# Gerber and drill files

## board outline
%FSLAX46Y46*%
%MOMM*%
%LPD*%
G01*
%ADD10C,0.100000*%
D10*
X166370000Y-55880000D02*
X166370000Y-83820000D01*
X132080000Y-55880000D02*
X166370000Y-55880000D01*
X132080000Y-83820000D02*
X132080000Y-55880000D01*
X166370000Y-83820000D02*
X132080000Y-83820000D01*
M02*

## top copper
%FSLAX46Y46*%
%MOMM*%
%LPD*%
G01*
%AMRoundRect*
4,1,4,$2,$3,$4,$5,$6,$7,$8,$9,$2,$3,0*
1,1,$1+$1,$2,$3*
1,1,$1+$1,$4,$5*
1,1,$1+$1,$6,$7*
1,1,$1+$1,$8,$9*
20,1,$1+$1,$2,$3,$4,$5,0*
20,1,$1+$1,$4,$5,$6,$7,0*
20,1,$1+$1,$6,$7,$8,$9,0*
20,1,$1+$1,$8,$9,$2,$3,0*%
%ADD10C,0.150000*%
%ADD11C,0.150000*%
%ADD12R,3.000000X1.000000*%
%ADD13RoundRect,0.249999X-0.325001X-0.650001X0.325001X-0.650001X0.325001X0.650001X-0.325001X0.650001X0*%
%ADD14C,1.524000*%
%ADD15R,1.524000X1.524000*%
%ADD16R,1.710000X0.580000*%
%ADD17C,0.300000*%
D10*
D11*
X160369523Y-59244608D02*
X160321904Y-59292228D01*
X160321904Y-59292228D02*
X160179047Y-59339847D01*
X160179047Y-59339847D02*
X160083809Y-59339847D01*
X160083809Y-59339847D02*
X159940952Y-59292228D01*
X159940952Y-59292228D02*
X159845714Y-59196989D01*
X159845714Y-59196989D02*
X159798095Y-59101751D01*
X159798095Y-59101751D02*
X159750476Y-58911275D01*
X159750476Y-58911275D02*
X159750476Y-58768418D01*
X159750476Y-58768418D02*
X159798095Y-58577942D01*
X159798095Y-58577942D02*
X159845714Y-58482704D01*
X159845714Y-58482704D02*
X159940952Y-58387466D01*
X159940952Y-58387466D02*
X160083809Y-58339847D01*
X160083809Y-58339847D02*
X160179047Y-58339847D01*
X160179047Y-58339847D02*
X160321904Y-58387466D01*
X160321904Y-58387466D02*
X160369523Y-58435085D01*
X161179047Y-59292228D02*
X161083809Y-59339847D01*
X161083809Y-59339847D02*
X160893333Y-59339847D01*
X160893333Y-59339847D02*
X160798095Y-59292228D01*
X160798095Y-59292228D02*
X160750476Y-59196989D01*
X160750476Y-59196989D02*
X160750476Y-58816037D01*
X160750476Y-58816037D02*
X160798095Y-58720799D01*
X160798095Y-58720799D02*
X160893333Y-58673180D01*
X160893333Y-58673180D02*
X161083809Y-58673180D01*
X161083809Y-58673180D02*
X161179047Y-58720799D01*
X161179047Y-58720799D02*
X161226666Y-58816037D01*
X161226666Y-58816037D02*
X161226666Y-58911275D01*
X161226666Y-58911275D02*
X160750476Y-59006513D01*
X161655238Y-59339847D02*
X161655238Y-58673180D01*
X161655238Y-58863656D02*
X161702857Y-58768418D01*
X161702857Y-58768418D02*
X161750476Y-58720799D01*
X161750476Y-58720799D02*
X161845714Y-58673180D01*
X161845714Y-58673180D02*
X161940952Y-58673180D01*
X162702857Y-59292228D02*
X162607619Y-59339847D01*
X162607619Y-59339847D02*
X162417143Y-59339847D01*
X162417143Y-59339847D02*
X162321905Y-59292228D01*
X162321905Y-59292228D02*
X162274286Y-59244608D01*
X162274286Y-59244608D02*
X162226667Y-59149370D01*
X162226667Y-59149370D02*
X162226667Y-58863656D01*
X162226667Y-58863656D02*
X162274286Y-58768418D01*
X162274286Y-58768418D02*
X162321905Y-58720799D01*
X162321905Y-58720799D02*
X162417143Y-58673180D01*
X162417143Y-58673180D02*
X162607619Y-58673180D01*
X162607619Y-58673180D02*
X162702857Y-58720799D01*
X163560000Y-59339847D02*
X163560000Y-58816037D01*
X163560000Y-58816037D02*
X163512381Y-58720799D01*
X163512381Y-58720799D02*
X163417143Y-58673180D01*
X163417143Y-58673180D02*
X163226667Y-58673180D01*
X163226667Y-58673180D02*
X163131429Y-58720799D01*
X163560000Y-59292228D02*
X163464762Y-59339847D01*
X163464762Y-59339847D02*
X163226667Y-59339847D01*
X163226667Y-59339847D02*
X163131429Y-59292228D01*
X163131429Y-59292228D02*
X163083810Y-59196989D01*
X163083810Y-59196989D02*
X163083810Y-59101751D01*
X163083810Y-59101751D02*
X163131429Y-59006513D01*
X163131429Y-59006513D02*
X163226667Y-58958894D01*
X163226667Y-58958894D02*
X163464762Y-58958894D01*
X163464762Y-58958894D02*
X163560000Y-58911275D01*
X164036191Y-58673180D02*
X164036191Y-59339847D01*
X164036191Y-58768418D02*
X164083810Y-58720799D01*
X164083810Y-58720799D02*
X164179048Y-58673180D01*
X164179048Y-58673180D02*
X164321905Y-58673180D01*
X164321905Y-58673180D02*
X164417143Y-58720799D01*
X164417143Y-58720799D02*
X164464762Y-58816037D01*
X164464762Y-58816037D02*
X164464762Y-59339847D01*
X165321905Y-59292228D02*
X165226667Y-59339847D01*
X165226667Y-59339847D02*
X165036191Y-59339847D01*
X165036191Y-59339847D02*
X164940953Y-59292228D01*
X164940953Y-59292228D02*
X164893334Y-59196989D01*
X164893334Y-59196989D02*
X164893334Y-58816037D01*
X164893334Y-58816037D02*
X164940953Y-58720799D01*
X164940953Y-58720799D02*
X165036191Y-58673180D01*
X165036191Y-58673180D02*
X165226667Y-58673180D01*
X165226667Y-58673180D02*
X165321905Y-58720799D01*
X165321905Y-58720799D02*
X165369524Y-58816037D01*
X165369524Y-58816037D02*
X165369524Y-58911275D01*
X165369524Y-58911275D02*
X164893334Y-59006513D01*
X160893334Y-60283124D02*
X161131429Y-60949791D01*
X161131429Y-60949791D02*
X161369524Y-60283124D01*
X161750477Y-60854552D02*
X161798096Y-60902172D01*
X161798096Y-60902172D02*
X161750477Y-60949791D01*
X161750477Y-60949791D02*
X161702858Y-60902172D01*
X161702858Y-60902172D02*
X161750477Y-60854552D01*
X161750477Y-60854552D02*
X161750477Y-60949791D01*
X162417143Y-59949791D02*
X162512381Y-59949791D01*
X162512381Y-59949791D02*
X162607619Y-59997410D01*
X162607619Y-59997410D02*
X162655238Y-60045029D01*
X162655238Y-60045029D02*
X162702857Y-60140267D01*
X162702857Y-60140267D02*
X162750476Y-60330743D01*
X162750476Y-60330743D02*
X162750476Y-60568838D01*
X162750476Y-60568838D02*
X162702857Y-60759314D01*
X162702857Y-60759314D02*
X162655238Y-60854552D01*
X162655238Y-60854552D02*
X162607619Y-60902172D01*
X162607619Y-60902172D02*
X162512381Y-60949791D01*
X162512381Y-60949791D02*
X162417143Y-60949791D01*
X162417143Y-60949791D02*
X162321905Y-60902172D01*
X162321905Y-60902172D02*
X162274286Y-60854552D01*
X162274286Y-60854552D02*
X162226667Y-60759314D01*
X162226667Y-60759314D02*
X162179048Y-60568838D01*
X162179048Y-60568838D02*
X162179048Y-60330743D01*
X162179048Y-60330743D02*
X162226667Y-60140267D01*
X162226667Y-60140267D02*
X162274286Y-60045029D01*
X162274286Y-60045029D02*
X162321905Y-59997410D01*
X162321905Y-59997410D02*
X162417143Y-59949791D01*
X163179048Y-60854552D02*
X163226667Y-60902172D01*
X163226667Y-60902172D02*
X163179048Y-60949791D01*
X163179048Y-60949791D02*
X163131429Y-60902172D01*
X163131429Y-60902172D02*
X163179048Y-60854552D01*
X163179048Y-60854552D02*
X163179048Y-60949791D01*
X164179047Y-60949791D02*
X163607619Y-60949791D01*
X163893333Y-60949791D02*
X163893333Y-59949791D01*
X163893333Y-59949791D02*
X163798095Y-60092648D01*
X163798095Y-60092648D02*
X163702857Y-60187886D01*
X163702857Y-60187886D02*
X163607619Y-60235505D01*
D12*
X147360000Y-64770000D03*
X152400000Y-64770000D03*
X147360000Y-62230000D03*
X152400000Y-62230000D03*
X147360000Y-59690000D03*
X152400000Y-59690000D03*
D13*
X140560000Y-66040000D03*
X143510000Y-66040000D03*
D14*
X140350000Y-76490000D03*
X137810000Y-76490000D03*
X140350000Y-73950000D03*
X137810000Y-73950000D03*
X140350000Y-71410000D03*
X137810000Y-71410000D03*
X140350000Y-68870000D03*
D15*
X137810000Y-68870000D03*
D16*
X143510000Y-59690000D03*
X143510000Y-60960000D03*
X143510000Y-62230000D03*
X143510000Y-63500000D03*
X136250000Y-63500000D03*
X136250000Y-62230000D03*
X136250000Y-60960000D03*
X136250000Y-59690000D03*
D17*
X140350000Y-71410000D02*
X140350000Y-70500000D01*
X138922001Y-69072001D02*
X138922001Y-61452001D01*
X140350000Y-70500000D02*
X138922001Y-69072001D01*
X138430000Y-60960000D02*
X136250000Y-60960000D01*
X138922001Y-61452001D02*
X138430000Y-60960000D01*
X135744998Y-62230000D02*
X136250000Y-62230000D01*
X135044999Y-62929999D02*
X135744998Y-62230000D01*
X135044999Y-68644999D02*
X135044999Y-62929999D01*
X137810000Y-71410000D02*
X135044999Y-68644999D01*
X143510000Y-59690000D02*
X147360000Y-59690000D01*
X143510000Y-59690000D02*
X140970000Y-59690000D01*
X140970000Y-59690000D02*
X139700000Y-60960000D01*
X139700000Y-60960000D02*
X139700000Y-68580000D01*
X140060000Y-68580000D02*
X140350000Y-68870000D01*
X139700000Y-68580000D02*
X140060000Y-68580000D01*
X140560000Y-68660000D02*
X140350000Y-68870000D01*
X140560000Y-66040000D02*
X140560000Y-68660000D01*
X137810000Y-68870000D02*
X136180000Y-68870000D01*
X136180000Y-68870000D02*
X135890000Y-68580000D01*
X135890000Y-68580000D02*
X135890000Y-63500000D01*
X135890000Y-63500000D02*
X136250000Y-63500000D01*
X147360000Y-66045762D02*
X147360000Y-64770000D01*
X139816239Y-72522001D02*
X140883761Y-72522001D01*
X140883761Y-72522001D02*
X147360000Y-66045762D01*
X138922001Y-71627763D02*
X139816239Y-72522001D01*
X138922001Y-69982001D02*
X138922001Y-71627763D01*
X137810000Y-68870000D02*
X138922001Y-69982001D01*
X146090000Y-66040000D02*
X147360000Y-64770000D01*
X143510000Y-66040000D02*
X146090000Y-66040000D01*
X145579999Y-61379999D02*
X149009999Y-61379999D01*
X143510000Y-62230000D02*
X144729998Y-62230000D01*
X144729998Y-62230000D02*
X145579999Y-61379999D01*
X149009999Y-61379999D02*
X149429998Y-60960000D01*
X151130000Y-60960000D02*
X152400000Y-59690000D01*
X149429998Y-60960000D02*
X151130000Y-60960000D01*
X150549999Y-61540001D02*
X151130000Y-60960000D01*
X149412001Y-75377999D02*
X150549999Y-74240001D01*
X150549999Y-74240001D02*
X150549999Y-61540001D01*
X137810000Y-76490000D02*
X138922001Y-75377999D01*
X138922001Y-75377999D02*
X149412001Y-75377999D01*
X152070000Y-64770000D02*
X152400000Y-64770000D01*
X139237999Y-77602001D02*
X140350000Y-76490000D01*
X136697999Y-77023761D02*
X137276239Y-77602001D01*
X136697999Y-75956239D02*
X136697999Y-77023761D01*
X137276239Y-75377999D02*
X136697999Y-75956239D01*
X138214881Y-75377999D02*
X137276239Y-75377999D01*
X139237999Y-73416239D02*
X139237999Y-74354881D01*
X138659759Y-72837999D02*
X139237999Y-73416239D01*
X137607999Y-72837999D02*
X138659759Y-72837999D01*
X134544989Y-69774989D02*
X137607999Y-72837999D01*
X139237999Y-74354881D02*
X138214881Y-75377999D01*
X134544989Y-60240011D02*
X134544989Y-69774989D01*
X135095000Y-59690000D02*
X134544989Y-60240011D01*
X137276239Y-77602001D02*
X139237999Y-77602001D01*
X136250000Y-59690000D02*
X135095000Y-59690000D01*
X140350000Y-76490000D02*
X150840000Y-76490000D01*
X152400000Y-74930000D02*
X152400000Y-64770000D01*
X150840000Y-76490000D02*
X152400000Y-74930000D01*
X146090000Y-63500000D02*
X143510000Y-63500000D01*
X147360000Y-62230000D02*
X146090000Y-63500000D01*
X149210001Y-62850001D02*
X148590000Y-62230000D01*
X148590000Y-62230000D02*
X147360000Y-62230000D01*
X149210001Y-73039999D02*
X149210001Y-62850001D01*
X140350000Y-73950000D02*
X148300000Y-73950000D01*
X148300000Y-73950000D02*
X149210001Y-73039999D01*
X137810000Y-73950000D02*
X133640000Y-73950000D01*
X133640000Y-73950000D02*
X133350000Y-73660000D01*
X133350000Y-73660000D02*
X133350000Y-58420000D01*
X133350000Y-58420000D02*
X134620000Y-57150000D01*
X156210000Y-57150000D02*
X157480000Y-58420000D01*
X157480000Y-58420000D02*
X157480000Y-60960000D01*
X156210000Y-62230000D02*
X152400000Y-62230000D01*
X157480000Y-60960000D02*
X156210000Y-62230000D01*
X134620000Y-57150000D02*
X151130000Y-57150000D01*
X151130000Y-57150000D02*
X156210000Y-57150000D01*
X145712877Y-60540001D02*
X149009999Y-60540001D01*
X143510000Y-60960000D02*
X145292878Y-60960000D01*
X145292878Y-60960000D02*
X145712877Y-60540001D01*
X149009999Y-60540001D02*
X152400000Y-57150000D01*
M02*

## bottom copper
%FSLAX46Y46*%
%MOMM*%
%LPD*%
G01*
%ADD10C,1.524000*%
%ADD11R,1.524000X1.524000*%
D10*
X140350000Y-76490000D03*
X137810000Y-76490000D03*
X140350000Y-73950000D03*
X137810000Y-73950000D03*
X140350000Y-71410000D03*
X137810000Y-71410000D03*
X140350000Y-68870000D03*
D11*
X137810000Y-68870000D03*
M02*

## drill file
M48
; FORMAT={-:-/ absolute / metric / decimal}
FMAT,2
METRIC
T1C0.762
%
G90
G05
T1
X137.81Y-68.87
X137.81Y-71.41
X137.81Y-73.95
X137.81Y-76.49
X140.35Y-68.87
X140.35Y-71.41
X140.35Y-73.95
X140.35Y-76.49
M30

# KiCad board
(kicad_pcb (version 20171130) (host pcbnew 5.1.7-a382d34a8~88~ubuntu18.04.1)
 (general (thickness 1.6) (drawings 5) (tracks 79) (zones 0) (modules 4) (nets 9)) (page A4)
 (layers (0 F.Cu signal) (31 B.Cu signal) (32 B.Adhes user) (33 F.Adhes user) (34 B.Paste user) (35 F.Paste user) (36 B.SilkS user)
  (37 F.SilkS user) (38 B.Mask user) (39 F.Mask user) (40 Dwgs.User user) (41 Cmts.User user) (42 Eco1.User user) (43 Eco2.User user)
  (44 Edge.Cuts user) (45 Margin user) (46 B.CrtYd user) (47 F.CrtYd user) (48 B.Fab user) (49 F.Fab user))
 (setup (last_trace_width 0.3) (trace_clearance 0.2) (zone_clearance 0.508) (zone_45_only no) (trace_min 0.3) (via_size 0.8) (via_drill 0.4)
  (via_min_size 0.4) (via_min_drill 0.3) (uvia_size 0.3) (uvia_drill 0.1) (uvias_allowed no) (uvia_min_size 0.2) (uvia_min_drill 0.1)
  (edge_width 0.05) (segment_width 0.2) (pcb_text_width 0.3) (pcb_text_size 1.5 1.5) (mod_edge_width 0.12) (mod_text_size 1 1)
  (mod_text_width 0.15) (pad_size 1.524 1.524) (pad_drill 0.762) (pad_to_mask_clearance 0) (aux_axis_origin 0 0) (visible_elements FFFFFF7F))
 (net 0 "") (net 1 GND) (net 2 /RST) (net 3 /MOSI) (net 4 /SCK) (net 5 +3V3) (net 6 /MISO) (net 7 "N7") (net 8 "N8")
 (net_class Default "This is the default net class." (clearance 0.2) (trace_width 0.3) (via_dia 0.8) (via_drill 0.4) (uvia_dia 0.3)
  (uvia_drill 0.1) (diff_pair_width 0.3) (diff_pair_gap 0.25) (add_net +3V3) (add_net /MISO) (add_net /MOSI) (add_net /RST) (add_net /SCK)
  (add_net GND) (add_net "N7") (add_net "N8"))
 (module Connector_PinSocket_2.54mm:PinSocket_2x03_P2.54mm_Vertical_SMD (layer F.Cu) (at 149.88 62.23)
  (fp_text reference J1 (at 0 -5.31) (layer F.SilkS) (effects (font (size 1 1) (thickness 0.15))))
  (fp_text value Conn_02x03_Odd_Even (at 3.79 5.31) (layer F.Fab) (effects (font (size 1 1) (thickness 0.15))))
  (pad 6 smd rect (at -2.52 2.54) (size 3 1) (layers F.Cu F.Paste F.Mask) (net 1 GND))
  (pad 5 smd rect (at 2.52 2.54) (size 3 1) (layers F.Cu F.Paste F.Mask) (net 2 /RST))
  (pad 4 smd rect (at -2.52 0) (size 3 1) (layers F.Cu F.Paste F.Mask) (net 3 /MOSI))
  (pad 3 smd rect (at 2.52 0) (size 3 1) (layers F.Cu F.Paste F.Mask) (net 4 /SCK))
  (pad 2 smd rect (at -2.52 -2.54) (size 3 1) (layers F.Cu F.Paste F.Mask) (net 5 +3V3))
  (pad 1 smd rect (at 2.52 -2.54) (size 3 1) (layers F.Cu F.Paste F.Mask) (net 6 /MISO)))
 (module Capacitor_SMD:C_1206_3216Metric (layer F.Cu) (at 142.035 66.04)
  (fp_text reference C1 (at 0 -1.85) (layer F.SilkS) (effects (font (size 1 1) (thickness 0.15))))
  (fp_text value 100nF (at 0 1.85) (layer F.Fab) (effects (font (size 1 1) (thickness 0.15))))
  (pad 1 smd roundrect (at -1.475 0) (size 1.15 1.8) (layers F.Cu F.Paste F.Mask) (roundrect_rratio 0.2173904347826087) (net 5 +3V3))
  (pad 2 smd roundrect (at 1.475 0) (size 1.15 1.8) (layers F.Cu F.Paste F.Mask) (roundrect_rratio 0.2173904347826087) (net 1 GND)))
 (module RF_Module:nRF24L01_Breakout (layer F.Cu) (at 137.81 68.87)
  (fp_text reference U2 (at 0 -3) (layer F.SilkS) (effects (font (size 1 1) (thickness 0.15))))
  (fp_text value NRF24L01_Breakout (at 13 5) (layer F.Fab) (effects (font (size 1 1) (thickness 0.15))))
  (pad 8 thru_hole circle (at 2.54 7.62) (size 1.524 1.524) (drill 0.762) (layers *.Cu *.Mask) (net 2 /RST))
  (pad 7 thru_hole circle (at 0 7.62) (size 1.524 1.524) (drill 0.762) (layers *.Cu *.Mask) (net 6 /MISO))
  (pad 6 thru_hole circle (at 2.54 5.08) (size 1.524 1.524) (drill 0.762) (layers *.Cu *.Mask) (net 3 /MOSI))
  (pad 5 thru_hole circle (at 0 5.08) (size 1.524 1.524) (drill 0.762) (layers *.Cu *.Mask) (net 4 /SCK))
  (pad 4 thru_hole circle (at 2.54 2.54) (size 1.524 1.524) (drill 0.762) (layers *.Cu *.Mask) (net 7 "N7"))
  (pad 3 thru_hole circle (at 0 2.54) (size 1.524 1.524) (drill 0.762) (layers *.Cu *.Mask) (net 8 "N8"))
  (pad 2 thru_hole circle (at 2.54 0) (size 1.524 1.524) (drill 0.762) (layers *.Cu *.Mask) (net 5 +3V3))
  (pad 1 thru_hole rect (at 0 0) (size 1.524 1.524) (drill 0.762) (layers *.Cu *.Mask) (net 1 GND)))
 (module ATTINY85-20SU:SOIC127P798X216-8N (layer F.Cu) (at 139.88 61.595)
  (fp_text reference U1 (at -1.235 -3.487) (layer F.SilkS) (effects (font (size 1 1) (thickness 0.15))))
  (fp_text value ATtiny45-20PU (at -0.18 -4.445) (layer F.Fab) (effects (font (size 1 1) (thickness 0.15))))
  (pad 8 smd rect (at 3.63 -1.905) (size 1.71 0.58) (layers F.Cu F.Paste F.Mask) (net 5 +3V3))
  (pad 7 smd rect (at 3.63 -0.635) (size 1.71 0.58) (layers F.Cu F.Paste F.Mask) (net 4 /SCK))
  (pad 6 smd rect (at 3.63 0.635) (size 1.71 0.58) (layers F.Cu F.Paste F.Mask) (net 6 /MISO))
  (pad 5 smd rect (at 3.63 1.905) (size 1.71 0.58) (layers F.Cu F.Paste F.Mask) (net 3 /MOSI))
  (pad 4 smd rect (at -3.63 1.905) (size 1.71 0.58) (layers F.Cu F.Paste F.Mask) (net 1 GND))
  (pad 3 smd rect (at -3.63 0.635) (size 1.71 0.58) (layers F.Cu F.Paste F.Mask) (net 8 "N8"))
  (pad 2 smd rect (at -3.63 -0.635) (size 1.71 0.58) (layers F.Cu F.Paste F.Mask) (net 7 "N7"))
  (pad 1 smd rect (at -3.63 -1.905) (size 1.71 0.58) (layers F.Cu F.Paste F.Mask) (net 2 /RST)))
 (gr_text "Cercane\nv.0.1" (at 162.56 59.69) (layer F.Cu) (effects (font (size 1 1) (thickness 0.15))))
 (gr_line (start 166.37 55.88) (end 166.37 83.82) (layer Edge.Cuts) (width 0.1))
 (gr_line (start 132.08 55.88) (end 166.37 55.88) (layer Edge.Cuts) (width 0.1))
 (gr_line (start 132.08 83.82) (end 132.08 55.88) (layer Edge.Cuts) (width 0.1))
 (gr_line (start 166.37 83.82) (end 132.08 83.82) (layer Edge.Cuts) (width 0.1))
 (segment (start 140.35 71.41) (end 140.35 70.5) (width 0.3) (layer F.Cu) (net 7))
 (segment (start 138.922001 69.072001) (end 138.922001 61.452001) (width 0.3) (layer F.Cu) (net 7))
 (segment (start 140.35 70.5) (end 138.922001 69.072001) (width 0.3) (layer F.Cu) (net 7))
 (segment (start 138.43 60.96) (end 136.25 60.96) (width 0.3) (layer F.Cu) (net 7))
 (segment (start 138.922001 61.452001) (end 138.43 60.96) (width 0.3) (layer F.Cu) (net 7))
 (segment (start 135.744998 62.23) (end 136.25 62.23) (width 0.3) (layer F.Cu) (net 8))
 (segment (start 135.044999 62.929999) (end 135.744998 62.23) (width 0.3) (layer F.Cu) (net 8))
 (segment (start 135.044999 68.644999) (end 135.044999 62.929999) (width 0.3) (layer F.Cu) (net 8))
 (segment (start 137.81 71.41) (end 135.044999 68.644999) (width 0.3) (layer F.Cu) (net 8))
 (segment (start 143.51 59.69) (end 147.36 59.69) (width 0.3) (layer F.Cu) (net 5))
 (segment (start 143.51 59.69) (end 140.97 59.69) (width 0.3) (layer F.Cu) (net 5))
 (segment (start 140.97 59.69) (end 139.7 60.96) (width 0.3) (layer F.Cu) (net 5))
 (segment (start 139.7 60.96) (end 139.7 68.58) (width 0.3) (layer F.Cu) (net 5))
 (segment (start 140.06 68.58) (end 140.35 68.87) (width 0.3) (layer F.Cu) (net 5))
 (segment (start 139.7 68.58) (end 140.06 68.58) (width 0.3) (layer F.Cu) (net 5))
 (segment (start 140.56 68.66) (end 140.35 68.87) (width 0.3) (layer F.Cu) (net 5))
 (segment (start 140.56 66.04) (end 140.56 68.66) (width 0.3) (layer F.Cu) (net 5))
 (segment (start 137.81 68.87) (end 136.18 68.87) (width 0.3) (layer F.Cu) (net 1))
 (segment (start 136.18 68.87) (end 135.89 68.58) (width 0.3) (layer F.Cu) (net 1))
 (segment (start 135.89 68.58) (end 135.89 63.5) (width 0.3) (layer F.Cu) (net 1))
 (segment (start 135.89 63.5) (end 136.25 63.5) (width 0.3) (layer F.Cu) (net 1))
 (segment (start 147.36 66.045762) (end 147.36 64.77) (width 0.3) (layer F.Cu) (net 1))
 (segment (start 139.816239 72.522001) (end 140.883761 72.522001) (width 0.3) (layer F.Cu) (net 1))
 (segment (start 140.883761 72.522001) (end 147.36 66.045762) (width 0.3) (layer F.Cu) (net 1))
 (segment (start 138.922001 71.627763) (end 139.816239 72.522001) (width 0.3) (layer F.Cu) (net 1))
 (segment (start 138.922001 69.982001) (end 138.922001 71.627763) (width 0.3) (layer F.Cu) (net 1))
 (segment (start 137.81 68.87) (end 138.922001 69.982001) (width 0.3) (layer F.Cu) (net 1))
 (segment (start 146.09 66.04) (end 147.36 64.77) (width 0.3) (layer F.Cu) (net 1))
 (segment (start 143.51 66.04) (end 146.09 66.04) (width 0.3) (layer F.Cu) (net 1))
 (segment (start 145.579999 61.379999) (end 149.009999 61.379999) (width 0.3) (layer F.Cu) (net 6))
 (segment (start 143.51 62.23) (end 144.729998 62.23) (width 0.3) (layer F.Cu) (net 6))
 (segment (start 144.729998 62.23) (end 145.579999 61.379999) (width 0.3) (layer F.Cu) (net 6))
 (segment (start 149.009999 61.379999) (end 149.429998 60.96) (width 0.3) (layer F.Cu) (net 6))
 (segment (start 151.13 60.96) (end 152.4 59.69) (width 0.3) (layer F.Cu) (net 6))
 (segment (start 149.429998 60.96) (end 151.13 60.96) (width 0.3) (layer F.Cu) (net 6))
 (segment (start 150.549999 61.540001) (end 151.13 60.96) (width 0.3) (layer F.Cu) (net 6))
 (segment (start 149.412001 75.377999) (end 150.549999 74.240001) (width 0.3) (layer F.Cu) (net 6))
 (segment (start 150.549999 74.240001) (end 150.549999 61.540001) (width 0.3) (layer F.Cu) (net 6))
 (segment (start 137.81 76.49) (end 138.922001 75.377999) (width 0.3) (layer F.Cu) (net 6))
 (segment (start 138.922001 75.377999) (end 149.412001 75.377999) (width 0.3) (layer F.Cu) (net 6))
 (segment (start 152.07 64.77) (end 152.4 64.77) (width 0.3) (layer F.Cu) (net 2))
 (segment (start 139.237999 77.602001) (end 140.35 76.49) (width 0.3) (layer F.Cu) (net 2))
 (segment (start 136.697999 77.023761) (end 137.276239 77.602001) (width 0.3) (layer F.Cu) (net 2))
 (segment (start 136.697999 75.956239) (end 136.697999 77.023761) (width 0.3) (layer F.Cu) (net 2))
 (segment (start 137.276239 75.377999) (end 136.697999 75.956239) (width 0.3) (layer F.Cu) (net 2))
 (segment (start 138.214881 75.377999) (end 137.276239 75.377999) (width 0.3) (layer F.Cu) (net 2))
 (segment (start 139.237999 73.416239) (end 139.237999 74.354881) (width 0.3) (layer F.Cu) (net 2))
 (segment (start 138.659759 72.837999) (end 139.237999 73.416239) (width 0.3) (layer F.Cu) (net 2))
 (segment (start 137.607999 72.837999) (end 138.659759 72.837999) (width 0.3) (layer F.Cu) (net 2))
 (segment (start 134.544989 69.774989) (end 137.607999 72.837999) (width 0.3) (layer F.Cu) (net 2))
 (segment (start 139.237999 74.354881) (end 138.214881 75.377999) (width 0.3) (layer F.Cu) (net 2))
 (segment (start 134.544989 60.240011) (end 134.544989 69.774989) (width 0.3) (layer F.Cu) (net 2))
 (segment (start 135.095 59.69) (end 134.544989 60.240011) (width 0.3) (layer F.Cu) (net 2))
 (segment (start 137.276239 77.602001) (end 139.237999 77.602001) (width 0.3) (layer F.Cu) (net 2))
 (segment (start 136.25 59.69) (end 135.095 59.69) (width 0.3) (layer F.Cu) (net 2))
 (segment (start 140.35 76.49) (end 150.84 76.49) (width 0.3) (layer F.Cu) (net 2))
 (segment (start 152.4 74.93) (end 152.4 64.77) (width 0.3) (layer F.Cu) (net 2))
 (segment (start 150.84 76.49) (end 152.4 74.93) (width 0.3) (layer F.Cu) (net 2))
 (segment (start 146.09 63.5) (end 143.51 63.5) (width 0.3) (layer F.Cu) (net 3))
 (segment (start 147.36 62.23) (end 146.09 63.5) (width 0.3) (layer F.Cu) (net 3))
 (segment (start 149.210001 62.850001) (end 148.59 62.23) (width 0.3) (layer F.Cu) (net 3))
 (segment (start 148.59 62.23) (end 147.36 62.23) (width 0.3) (layer F.Cu) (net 3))
 (segment (start 149.210001 73.039999) (end 149.210001 62.850001) (width 0.3) (layer F.Cu) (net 3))
 (segment (start 140.35 73.95) (end 148.3 73.95) (width 0.3) (layer F.Cu) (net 3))
 (segment (start 148.3 73.95) (end 149.210001 73.039999) (width 0.3) (layer F.Cu) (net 3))
 (segment (start 137.81 73.95) (end 133.64 73.95) (width 0.3) (layer F.Cu) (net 4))
 (segment (start 133.64 73.95) (end 133.35 73.66) (width 0.3) (layer F.Cu) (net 4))
 (segment (start 133.35 73.66) (end 133.35 58.42) (width 0.3) (layer F.Cu) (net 4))
 (segment (start 133.35 58.42) (end 134.62 57.15) (width 0.3) (layer F.Cu) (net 4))
 (segment (start 156.21 57.15) (end 157.48 58.42) (width 0.3) (layer F.Cu) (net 4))
 (segment (start 157.48 58.42) (end 157.48 60.96) (width 0.3) (layer F.Cu) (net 4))
 (segment (start 156.21 62.23) (end 152.4 62.23) (width 0.3) (layer F.Cu) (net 4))
 (segment (start 157.48 60.96) (end 156.21 62.23) (width 0.3) (layer F.Cu) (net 4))
 (segment (start 134.62 57.15) (end 151.13 57.15) (width 0.3) (layer F.Cu) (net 4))
 (segment (start 151.13 57.15) (end 156.21 57.15) (width 0.3) (layer F.Cu) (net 4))
 (segment (start 145.712877 60.540001) (end 149.009999 60.540001) (width 0.3) (layer F.Cu) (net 4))
 (segment (start 143.51 60.96) (end 145.292878 60.96) (width 0.3) (layer F.Cu) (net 4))
 (segment (start 145.292878 60.96) (end 145.712877 60.540001) (width 0.3) (layer F.Cu) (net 4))
 (segment (start 149.009999 60.540001) (end 152.4 57.15) (width 0.3) (layer F.Cu) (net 4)))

